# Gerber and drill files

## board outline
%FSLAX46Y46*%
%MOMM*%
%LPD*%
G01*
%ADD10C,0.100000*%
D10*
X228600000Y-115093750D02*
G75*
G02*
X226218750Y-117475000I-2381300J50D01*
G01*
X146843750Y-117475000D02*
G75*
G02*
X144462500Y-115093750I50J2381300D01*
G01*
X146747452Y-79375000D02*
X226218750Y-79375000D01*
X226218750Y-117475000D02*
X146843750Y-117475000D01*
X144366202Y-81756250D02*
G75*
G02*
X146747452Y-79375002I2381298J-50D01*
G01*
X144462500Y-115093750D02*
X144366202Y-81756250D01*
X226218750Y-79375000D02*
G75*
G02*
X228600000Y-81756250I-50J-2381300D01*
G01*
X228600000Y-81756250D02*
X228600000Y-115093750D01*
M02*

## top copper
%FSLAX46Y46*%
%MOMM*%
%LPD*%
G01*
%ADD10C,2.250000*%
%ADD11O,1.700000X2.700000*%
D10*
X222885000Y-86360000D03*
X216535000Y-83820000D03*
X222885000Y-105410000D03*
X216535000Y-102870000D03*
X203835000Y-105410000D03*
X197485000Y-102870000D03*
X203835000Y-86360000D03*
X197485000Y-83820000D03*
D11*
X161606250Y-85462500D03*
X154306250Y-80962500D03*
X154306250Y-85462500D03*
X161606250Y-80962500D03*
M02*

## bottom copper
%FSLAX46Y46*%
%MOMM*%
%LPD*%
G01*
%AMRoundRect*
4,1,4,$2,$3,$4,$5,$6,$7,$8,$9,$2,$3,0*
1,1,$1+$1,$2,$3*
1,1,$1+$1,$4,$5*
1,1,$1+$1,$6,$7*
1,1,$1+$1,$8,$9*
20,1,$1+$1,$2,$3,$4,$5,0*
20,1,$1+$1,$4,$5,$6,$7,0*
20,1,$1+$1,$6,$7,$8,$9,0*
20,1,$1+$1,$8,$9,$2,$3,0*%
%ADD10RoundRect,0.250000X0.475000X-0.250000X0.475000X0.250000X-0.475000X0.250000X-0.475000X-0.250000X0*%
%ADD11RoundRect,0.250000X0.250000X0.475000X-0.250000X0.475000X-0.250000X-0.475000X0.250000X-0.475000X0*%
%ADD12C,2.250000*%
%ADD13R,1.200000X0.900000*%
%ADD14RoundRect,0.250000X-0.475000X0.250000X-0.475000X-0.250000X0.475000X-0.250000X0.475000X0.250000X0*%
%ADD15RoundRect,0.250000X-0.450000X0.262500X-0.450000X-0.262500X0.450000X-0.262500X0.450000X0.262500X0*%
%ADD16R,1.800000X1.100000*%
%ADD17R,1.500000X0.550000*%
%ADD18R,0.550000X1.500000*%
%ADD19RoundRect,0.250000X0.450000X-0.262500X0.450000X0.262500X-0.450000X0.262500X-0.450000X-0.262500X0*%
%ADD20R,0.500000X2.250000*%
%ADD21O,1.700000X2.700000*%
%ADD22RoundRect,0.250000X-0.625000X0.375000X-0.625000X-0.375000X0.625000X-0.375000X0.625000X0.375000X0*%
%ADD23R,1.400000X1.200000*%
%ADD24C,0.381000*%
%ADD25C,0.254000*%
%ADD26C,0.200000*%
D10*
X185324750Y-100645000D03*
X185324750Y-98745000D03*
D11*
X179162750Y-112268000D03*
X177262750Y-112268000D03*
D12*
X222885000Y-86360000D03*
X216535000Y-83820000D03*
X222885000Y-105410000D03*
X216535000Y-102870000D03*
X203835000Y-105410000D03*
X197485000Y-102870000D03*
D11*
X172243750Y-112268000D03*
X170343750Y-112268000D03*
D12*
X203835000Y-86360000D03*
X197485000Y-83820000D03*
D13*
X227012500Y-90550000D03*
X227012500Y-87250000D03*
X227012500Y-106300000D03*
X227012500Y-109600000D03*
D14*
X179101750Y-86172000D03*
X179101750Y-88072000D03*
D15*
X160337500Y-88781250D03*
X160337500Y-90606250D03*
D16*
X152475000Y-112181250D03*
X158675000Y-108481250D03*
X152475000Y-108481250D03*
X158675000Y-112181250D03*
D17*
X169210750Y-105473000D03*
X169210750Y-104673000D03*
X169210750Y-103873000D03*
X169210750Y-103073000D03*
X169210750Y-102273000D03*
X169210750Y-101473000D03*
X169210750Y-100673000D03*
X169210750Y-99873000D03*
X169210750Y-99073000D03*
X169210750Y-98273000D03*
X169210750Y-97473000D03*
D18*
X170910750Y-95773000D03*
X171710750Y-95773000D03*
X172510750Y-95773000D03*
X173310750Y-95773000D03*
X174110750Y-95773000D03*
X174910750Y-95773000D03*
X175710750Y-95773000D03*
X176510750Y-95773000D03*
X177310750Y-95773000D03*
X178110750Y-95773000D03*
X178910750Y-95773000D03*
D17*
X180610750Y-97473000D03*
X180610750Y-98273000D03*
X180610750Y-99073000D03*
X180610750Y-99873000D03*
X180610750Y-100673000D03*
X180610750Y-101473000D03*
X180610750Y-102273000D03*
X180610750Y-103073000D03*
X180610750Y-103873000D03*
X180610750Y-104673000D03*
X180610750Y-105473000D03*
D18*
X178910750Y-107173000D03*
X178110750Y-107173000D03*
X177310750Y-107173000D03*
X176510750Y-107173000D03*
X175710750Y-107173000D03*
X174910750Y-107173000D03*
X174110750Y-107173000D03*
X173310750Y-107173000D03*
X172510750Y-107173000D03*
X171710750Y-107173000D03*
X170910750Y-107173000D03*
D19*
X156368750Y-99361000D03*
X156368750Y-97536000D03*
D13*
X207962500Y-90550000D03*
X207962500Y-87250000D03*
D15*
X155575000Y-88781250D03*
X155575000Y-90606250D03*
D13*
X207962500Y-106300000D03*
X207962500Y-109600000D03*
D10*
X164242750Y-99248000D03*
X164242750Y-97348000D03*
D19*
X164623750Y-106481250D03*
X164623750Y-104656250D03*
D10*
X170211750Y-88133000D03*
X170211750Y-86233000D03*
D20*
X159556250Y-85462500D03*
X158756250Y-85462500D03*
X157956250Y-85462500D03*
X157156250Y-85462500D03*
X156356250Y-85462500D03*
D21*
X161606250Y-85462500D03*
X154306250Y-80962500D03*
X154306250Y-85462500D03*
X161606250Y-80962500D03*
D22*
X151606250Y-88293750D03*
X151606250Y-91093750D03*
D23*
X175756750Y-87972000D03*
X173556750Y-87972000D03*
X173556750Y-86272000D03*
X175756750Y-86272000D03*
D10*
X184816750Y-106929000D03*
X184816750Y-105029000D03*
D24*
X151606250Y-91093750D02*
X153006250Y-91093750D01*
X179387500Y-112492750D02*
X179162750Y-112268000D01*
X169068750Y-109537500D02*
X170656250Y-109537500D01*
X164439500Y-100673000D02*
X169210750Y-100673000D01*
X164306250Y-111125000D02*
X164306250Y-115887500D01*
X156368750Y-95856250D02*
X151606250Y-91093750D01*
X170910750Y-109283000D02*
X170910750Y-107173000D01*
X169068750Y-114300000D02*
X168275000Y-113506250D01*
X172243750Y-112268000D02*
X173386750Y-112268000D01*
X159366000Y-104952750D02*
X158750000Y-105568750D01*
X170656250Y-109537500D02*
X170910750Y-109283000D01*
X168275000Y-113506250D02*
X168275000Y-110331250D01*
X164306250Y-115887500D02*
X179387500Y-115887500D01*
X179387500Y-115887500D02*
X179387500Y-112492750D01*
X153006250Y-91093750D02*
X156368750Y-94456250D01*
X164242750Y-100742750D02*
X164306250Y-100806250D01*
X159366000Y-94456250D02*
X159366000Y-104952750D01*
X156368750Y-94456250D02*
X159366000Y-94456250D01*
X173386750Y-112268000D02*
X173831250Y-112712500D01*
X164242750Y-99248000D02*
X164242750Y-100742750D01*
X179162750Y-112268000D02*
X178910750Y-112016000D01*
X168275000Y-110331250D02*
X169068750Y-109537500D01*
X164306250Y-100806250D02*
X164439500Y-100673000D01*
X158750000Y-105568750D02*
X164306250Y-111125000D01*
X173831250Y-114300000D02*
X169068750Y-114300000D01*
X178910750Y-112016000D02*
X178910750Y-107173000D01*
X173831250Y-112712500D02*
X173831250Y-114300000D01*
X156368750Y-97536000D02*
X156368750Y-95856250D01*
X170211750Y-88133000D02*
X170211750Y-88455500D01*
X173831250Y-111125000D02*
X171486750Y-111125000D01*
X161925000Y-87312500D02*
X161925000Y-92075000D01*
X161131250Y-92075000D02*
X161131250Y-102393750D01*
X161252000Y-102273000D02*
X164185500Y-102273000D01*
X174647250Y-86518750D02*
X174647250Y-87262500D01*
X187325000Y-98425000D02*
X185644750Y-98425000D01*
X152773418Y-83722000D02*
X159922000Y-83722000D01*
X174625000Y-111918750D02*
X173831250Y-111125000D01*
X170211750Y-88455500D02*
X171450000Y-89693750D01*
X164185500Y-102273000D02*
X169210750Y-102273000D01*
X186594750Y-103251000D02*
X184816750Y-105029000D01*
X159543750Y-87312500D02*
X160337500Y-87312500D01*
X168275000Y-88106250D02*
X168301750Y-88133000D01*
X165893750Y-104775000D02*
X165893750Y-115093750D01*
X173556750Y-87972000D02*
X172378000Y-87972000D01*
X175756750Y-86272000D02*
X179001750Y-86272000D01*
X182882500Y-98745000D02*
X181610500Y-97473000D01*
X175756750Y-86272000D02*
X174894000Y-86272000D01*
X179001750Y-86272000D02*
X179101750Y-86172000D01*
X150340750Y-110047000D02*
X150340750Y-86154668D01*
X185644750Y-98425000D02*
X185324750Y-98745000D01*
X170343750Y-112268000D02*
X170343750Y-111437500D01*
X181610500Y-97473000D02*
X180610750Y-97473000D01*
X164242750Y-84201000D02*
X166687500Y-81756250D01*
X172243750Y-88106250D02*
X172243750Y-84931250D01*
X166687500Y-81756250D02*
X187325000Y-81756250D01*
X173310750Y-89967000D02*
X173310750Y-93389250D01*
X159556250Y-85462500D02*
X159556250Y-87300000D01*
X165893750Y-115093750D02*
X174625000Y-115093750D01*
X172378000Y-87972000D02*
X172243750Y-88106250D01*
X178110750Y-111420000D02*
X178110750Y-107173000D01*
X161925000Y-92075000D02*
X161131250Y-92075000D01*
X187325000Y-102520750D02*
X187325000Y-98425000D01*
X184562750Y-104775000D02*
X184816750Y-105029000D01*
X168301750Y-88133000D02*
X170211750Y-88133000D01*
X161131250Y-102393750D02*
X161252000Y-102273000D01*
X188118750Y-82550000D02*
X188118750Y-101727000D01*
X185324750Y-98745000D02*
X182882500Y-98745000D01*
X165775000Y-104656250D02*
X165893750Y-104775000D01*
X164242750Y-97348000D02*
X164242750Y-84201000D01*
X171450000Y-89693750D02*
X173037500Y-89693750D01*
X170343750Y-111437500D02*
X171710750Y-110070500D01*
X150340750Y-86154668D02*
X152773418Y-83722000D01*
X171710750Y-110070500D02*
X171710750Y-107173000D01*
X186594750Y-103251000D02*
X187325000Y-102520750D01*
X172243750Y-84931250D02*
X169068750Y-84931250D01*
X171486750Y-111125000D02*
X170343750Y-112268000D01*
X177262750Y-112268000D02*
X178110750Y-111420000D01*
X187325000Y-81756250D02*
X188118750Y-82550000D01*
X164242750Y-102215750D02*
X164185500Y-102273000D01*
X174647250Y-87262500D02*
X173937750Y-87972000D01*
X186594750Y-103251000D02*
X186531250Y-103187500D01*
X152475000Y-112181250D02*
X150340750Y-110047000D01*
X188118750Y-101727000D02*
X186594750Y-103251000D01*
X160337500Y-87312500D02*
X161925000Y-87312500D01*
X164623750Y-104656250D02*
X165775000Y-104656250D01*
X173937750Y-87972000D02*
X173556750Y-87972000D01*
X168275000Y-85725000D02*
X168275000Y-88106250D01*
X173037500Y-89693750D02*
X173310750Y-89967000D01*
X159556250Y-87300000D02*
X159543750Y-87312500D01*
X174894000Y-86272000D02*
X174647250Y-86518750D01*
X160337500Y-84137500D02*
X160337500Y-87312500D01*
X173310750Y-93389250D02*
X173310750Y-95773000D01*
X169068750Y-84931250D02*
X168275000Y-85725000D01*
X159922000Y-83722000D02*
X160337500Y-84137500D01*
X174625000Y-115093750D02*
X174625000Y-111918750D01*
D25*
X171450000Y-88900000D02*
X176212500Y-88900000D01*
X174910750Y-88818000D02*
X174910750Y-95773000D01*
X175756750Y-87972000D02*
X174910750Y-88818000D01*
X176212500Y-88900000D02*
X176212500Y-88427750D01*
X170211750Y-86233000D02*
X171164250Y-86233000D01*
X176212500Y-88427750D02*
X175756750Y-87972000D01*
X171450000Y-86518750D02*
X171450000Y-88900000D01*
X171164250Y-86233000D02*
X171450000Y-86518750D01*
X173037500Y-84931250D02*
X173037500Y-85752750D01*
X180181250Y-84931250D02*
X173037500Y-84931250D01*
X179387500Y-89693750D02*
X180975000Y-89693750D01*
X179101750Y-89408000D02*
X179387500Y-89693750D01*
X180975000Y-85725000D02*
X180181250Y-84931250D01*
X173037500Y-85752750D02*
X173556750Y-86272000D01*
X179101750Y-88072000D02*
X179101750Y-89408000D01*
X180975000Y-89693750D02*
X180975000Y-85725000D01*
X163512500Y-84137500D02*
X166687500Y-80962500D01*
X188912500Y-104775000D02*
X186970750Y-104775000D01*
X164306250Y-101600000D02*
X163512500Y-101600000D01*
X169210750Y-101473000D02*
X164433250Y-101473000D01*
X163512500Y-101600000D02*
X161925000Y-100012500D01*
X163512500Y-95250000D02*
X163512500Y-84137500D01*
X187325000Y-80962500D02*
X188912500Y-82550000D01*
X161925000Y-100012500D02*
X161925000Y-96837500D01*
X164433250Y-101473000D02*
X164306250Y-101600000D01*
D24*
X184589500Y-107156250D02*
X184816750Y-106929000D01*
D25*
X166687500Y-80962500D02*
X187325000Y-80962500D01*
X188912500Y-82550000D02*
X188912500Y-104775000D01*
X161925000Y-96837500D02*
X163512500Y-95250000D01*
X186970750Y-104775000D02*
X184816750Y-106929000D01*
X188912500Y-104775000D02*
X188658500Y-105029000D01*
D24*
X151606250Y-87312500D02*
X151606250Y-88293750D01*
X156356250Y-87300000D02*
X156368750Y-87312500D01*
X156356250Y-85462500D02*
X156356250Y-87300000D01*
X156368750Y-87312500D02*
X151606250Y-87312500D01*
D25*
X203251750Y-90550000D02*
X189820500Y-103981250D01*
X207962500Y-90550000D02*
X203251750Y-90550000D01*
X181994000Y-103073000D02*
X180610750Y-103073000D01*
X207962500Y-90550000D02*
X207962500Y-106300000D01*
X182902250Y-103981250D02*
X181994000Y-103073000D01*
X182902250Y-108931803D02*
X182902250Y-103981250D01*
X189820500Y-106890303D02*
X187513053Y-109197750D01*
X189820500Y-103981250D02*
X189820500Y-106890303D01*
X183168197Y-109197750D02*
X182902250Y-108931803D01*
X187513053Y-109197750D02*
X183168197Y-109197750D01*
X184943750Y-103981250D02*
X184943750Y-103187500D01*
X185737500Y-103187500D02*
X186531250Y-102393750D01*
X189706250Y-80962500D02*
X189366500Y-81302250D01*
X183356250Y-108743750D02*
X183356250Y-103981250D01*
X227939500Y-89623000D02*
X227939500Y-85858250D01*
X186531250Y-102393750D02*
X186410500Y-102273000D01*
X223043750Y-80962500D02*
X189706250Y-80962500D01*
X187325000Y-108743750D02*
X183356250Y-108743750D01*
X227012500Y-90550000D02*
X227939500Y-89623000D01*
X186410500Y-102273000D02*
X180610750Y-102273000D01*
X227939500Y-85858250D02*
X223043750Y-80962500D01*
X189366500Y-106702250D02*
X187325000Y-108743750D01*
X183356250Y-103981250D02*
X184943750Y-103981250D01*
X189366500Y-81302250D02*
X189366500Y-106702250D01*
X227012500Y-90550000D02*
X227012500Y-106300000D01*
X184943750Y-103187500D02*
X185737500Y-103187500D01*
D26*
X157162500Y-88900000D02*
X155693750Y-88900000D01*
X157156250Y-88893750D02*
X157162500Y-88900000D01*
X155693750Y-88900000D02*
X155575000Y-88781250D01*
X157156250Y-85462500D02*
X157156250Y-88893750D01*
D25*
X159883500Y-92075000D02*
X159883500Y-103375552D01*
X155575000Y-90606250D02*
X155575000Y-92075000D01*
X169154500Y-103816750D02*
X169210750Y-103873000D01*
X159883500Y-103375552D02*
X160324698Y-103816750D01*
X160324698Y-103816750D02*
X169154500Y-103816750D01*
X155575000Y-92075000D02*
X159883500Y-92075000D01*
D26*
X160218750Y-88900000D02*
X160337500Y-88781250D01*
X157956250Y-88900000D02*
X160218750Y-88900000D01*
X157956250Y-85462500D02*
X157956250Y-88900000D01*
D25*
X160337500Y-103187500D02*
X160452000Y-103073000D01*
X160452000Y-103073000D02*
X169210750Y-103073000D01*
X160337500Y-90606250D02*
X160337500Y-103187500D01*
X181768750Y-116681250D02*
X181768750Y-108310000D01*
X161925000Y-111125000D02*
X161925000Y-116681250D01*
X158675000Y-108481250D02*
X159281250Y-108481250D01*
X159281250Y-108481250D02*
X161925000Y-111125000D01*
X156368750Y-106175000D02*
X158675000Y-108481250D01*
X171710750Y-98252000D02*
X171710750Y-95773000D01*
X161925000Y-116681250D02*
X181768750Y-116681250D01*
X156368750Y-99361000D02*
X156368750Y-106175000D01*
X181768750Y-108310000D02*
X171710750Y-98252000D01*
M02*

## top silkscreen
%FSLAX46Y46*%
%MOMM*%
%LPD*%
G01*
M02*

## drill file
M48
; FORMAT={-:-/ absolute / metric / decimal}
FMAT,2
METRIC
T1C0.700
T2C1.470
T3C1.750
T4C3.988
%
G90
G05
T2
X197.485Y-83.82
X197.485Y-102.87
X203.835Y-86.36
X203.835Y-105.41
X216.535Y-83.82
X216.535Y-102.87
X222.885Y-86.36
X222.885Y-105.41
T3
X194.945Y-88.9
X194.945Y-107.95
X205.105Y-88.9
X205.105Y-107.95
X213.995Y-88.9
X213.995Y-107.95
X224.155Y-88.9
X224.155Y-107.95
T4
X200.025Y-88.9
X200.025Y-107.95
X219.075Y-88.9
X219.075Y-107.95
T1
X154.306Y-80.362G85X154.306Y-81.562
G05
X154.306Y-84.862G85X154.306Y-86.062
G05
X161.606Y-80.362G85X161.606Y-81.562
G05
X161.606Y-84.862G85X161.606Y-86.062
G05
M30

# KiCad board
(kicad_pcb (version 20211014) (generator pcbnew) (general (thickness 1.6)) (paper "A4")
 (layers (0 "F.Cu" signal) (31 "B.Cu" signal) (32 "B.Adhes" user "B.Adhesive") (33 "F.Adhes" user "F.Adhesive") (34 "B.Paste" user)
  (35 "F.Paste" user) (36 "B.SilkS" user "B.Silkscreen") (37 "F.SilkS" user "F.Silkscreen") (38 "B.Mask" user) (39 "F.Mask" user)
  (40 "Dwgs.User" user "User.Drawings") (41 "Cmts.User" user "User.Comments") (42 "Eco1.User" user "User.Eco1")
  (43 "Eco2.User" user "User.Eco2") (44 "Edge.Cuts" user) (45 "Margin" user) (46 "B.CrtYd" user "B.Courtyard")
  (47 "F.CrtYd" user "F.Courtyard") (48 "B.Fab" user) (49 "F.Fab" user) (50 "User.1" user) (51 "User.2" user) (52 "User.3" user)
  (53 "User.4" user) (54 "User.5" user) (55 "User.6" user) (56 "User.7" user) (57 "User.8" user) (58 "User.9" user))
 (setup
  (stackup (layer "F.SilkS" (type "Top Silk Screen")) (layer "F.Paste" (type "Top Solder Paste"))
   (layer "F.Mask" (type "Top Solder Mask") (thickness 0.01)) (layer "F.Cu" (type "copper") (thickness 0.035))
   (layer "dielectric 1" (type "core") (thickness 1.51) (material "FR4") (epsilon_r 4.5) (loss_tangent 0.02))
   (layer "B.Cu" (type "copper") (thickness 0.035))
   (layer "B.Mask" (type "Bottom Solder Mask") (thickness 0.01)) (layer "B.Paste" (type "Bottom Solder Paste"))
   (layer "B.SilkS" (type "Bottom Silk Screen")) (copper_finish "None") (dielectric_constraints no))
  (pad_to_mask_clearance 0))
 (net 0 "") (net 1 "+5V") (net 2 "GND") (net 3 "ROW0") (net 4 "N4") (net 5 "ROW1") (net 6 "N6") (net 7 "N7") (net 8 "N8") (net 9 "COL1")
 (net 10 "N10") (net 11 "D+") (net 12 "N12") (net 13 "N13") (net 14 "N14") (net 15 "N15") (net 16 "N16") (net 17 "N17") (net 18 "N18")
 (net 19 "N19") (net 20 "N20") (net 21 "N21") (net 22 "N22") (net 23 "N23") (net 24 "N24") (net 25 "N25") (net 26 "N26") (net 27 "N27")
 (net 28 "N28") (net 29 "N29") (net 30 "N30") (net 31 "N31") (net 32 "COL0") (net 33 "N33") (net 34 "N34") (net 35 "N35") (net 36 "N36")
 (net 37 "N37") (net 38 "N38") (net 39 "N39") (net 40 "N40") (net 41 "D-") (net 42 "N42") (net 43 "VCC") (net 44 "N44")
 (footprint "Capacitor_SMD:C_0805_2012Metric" (layer "B.Cu") (at 185.32475 99.695 90)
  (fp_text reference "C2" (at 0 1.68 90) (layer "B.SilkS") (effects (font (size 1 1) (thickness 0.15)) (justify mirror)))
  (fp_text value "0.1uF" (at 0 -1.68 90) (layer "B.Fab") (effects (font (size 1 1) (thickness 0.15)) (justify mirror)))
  (pad "1" smd roundrect (at -0.95 0 90) (size 1 1.45) (layers "B.Cu" "B.Paste" "B.Mask") (roundrect_rratio 0.25) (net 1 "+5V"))
  (pad "2" smd roundrect (at 0.95 0 90) (size 1 1.45) (layers "B.Cu" "B.Paste" "B.Mask") (roundrect_rratio 0.25) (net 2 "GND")))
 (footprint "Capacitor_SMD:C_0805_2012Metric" (layer "B.Cu") (at 178.21275 112.268 180)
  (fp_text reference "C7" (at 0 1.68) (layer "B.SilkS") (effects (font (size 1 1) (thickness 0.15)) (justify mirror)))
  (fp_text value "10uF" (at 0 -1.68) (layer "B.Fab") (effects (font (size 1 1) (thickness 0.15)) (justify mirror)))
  (pad "1" smd roundrect (at -0.95 0 180) (size 1 1.45) (layers "B.Cu" "B.Paste" "B.Mask") (roundrect_rratio 0.25) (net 1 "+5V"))
  (pad "2" smd roundrect (at 0.95 0 180) (size 1 1.45) (layers "B.Cu" "B.Paste" "B.Mask") (roundrect_rratio 0.25) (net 2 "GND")))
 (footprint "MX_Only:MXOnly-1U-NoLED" (layer "B.Cu") (at 219.075 88.9 180)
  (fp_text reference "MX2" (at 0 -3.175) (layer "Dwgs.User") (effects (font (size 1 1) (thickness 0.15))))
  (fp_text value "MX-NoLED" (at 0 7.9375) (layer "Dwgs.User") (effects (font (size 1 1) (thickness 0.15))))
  (pad "" np_thru_hole circle locked (at 0 0 180) (size 3.9878 3.9878) (drill 3.9878) (layers *.Cu *.Mask))
  (pad "" np_thru_hole circle locked (at -5.08 0 131.9004) (size 1.75 1.75) (drill 1.75) (layers *.Cu *.Mask))
  (pad "" np_thru_hole circle locked (at 5.08 0 131.9004) (size 1.75 1.75) (drill 1.75) (layers *.Cu *.Mask))
  (pad "1" thru_hole circle locked (at -3.81 2.54 180) (size 2.25 2.25) (drill 1.47) (layers *.Cu "F.Mask") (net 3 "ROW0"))
  (pad "2" thru_hole circle locked (at 2.54 5.08 180) (size 2.25 2.25) (drill 1.47) (layers *.Cu "F.Mask") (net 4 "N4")))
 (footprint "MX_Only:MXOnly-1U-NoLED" (layer "B.Cu") (at 219.075 107.95 180)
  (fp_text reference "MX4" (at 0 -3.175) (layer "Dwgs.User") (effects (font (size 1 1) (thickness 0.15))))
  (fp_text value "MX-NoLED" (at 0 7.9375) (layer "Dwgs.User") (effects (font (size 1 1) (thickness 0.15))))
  (pad "" np_thru_hole circle locked (at -5.08 0 131.9004) (size 1.75 1.75) (drill 1.75) (layers *.Cu *.Mask))
  (pad "" np_thru_hole circle locked (at 0 0 180) (size 3.9878 3.9878) (drill 3.9878) (layers *.Cu *.Mask))
  (pad "" np_thru_hole circle locked (at 5.08 0 131.9004) (size 1.75 1.75) (drill 1.75) (layers *.Cu *.Mask))
  (pad "1" thru_hole circle locked (at -3.81 2.54 180) (size 2.25 2.25) (drill 1.47) (layers *.Cu "F.Mask") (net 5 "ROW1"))
  (pad "2" thru_hole circle locked (at 2.54 5.08 180) (size 2.25 2.25) (drill 1.47) (layers *.Cu "F.Mask") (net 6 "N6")))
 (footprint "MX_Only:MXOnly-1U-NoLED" (layer "B.Cu") (at 200.025 107.95 180)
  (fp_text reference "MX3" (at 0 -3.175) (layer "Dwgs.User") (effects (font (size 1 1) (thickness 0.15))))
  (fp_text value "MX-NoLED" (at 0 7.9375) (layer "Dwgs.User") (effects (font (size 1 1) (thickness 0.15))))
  (pad "" np_thru_hole circle locked (at 5.08 0 131.9004) (size 1.75 1.75) (drill 1.75) (layers *.Cu *.Mask))
  (pad "" np_thru_hole circle locked (at 0 0 180) (size 3.9878 3.9878) (drill 3.9878) (layers *.Cu *.Mask))
  (pad "" np_thru_hole circle locked (at -5.08 0 131.9004) (size 1.75 1.75) (drill 1.75) (layers *.Cu *.Mask))
  (pad "1" thru_hole circle locked (at -3.81 2.54 180) (size 2.25 2.25) (drill 1.47) (layers *.Cu "F.Mask") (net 5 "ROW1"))
  (pad "2" thru_hole circle locked (at 2.54 5.08 180) (size 2.25 2.25) (drill 1.47) (layers *.Cu "F.Mask") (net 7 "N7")))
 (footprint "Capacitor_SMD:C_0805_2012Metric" (layer "B.Cu") (at 171.29375 112.268 180)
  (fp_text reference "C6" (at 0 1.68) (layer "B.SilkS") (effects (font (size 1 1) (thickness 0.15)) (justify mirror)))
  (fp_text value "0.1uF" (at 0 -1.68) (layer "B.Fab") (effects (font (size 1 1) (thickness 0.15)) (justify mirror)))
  (pad "1" smd roundrect (at -0.95 0 180) (size 1 1.45) (layers "B.Cu" "B.Paste" "B.Mask") (roundrect_rratio 0.25) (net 1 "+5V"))
  (pad "2" smd roundrect (at 0.95 0 180) (size 1 1.45) (layers "B.Cu" "B.Paste" "B.Mask") (roundrect_rratio 0.25) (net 2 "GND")))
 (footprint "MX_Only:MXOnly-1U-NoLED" (layer "B.Cu") (at 200.025 88.9 180)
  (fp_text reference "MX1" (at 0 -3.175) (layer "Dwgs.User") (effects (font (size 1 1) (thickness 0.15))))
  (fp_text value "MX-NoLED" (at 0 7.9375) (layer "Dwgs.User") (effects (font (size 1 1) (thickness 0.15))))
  (pad "" np_thru_hole circle locked (at 5.08 0 131.9004) (size 1.75 1.75) (drill 1.75) (layers *.Cu *.Mask))
  (pad "" np_thru_hole circle locked (at -5.08 0 131.9004) (size 1.75 1.75) (drill 1.75) (layers *.Cu *.Mask))
  (pad "" np_thru_hole circle locked (at 0 0 180) (size 3.9878 3.9878) (drill 3.9878) (layers *.Cu *.Mask))
  (pad "1" thru_hole circle locked (at -3.81 2.54 180) (size 2.25 2.25) (drill 1.47) (layers *.Cu "F.Mask") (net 3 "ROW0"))
  (pad "2" thru_hole circle locked (at 2.54 5.08 180) (size 2.25 2.25) (drill 1.47) (layers *.Cu "F.Mask") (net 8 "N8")))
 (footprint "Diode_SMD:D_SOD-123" (layer "B.Cu") (at 227.0125 88.9 90)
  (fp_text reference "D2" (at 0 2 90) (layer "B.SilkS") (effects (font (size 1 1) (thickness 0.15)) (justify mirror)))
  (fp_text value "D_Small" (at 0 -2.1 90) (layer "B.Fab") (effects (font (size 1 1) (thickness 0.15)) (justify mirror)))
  (pad "1" smd rect (at -1.65 0 90) (size 0.9 1.2) (layers "B.Cu" "B.Paste" "B.Mask") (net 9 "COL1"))
  (pad "2" smd rect (at 1.65 0 90) (size 0.9 1.2) (layers "B.Cu" "B.Paste" "B.Mask") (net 4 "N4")))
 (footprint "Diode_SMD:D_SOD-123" (layer "B.Cu") (at 227.0125 107.95 -90)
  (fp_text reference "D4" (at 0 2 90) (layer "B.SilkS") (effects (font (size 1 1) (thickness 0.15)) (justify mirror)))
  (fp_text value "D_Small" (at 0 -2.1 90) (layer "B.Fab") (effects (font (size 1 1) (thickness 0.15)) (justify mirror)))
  (pad "1" smd rect (at -1.65 0 270) (size 0.9 1.2) (layers "B.Cu" "B.Paste" "B.Mask") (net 9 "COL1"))
  (pad "2" smd rect (at 1.65 0 270) (size 0.9 1.2) (layers "B.Cu" "B.Paste" "B.Mask") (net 6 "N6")))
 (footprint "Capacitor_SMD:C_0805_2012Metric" (layer "B.Cu") (at 179.10175 87.122 -90)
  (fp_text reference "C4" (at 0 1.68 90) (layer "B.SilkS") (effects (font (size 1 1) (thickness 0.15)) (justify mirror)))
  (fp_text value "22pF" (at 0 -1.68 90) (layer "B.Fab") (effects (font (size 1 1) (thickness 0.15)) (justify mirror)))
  (pad "1" smd roundrect (at -0.95 0 270) (size 1 1.45) (layers "B.Cu" "B.Paste" "B.Mask") (roundrect_rratio 0.25) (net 2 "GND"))
  (pad "2" smd roundrect (at 0.95 0 270) (size 1 1.45) (layers "B.Cu" "B.Paste" "B.Mask") (roundrect_rratio 0.25) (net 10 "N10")))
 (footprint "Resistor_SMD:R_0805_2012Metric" (layer "B.Cu") (at 160.3375 89.69375 -90)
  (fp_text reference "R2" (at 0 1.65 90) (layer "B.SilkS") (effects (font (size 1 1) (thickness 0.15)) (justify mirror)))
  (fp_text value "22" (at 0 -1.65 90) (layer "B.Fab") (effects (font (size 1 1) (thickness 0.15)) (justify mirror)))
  (pad "1" smd roundrect (at -0.9125 0 270) (size 1.025 1.4) (layers "B.Cu" "B.Paste" "B.Mask") (roundrect_rratio 0.243902) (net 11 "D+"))
  (pad "2" smd roundrect (at 0.9125 0 270) (size 1.025 1.4) (layers "B.Cu" "B.Paste" "B.Mask") (roundrect_rratio 0.243902) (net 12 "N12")))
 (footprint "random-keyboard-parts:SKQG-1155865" (layer "B.Cu") (at 155.575 110.33125 180)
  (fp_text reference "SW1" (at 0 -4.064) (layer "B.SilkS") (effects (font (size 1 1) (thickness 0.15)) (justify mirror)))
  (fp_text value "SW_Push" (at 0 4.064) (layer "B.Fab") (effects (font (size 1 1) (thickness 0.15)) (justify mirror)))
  (pad "1" smd rect locked (at 3.1 -1.85 180) (size 1.8 1.1) (layers "B.Cu" "B.Paste" "B.Mask") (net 2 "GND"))
  (pad "2" smd rect locked (at -3.1 1.85 180) (size 1.8 1.1) (layers "B.Cu" "B.Paste" "B.Mask") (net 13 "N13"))
  (pad "3" smd rect locked (at 3.1 1.85 180) (size 1.8 1.1) (layers "B.Cu" "B.Paste" "B.Mask"))
  (pad "4" smd rect locked (at -3.1 -1.85 180) (size 1.8 1.1) (layers "B.Cu" "B.Paste" "B.Mask")))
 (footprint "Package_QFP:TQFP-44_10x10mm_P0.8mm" (layer "B.Cu") (at 174.91075 101.473)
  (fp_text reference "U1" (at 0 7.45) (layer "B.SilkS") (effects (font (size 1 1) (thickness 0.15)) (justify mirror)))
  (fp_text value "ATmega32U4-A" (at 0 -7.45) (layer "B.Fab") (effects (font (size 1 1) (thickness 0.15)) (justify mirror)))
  (pad "1" smd rect (at -5.7 4) (size 1.5 0.55) (layers "B.Cu" "B.Paste" "B.Mask") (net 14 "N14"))
  (pad "2" smd rect (at -5.7 3.2) (size 1.5 0.55) (layers "B.Cu" "B.Paste" "B.Mask") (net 1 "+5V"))
  (pad "3" smd rect (at -5.7 2.4) (size 1.5 0.55) (layers "B.Cu" "B.Paste" "B.Mask") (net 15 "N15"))
  (pad "4" smd rect (at -5.7 1.6) (size 1.5 0.55) (layers "B.Cu" "B.Paste" "B.Mask") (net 12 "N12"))
  (pad "5" smd rect (at -5.7 0.8) (size 1.5 0.55) (layers "B.Cu" "B.Paste" "B.Mask") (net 2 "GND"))
  (pad "6" smd rect (at -5.7 0) (size 1.5 0.55) (layers "B.Cu" "B.Paste" "B.Mask") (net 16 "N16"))
  (pad "7" smd rect (at -5.7 -0.8) (size 1.5 0.55) (layers "B.Cu" "B.Paste" "B.Mask") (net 1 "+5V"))
  (pad "8" smd rect (at -5.7 -1.6) (size 1.5 0.55) (layers "B.Cu" "B.Paste" "B.Mask") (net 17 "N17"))
  (pad "9" smd rect (at -5.7 -2.4) (size 1.5 0.55) (layers "B.Cu" "B.Paste" "B.Mask") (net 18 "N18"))
  (pad "10" smd rect (at -5.7 -3.2) (size 1.5 0.55) (layers "B.Cu" "B.Paste" "B.Mask") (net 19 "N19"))
  (pad "11" smd rect (at -5.7 -4) (size 1.5 0.55) (layers "B.Cu" "B.Paste" "B.Mask") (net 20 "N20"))
  (pad "12" smd rect (at -4 -5.7 270) (size 1.5 0.55) (layers "B.Cu" "B.Paste" "B.Mask") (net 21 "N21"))
  (pad "13" smd rect (at -3.2 -5.7 270) (size 1.5 0.55) (layers "B.Cu" "B.Paste" "B.Mask") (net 13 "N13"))
  (pad "14" smd rect (at -2.4 -5.7 270) (size 1.5 0.55) (layers "B.Cu" "B.Paste" "B.Mask") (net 1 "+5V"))
  (pad "15" smd rect (at -1.6 -5.7 270) (size 1.5 0.55) (layers "B.Cu" "B.Paste" "B.Mask") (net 2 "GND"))
  (pad "16" smd rect (at -0.8 -5.7 270) (size 1.5 0.55) (layers "B.Cu" "B.Paste" "B.Mask") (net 10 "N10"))
  (pad "17" smd rect (at 0 -5.7 270) (size 1.5 0.55) (layers "B.Cu" "B.Paste" "B.Mask") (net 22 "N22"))
  (pad "18" smd rect (at 0.8 -5.7 270) (size 1.5 0.55) (layers "B.Cu" "B.Paste" "B.Mask") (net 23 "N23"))
  (pad "19" smd rect (at 1.6 -5.7 270) (size 1.5 0.55) (layers "B.Cu" "B.Paste" "B.Mask") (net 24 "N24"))
  (pad "20" smd rect (at 2.4 -5.7 270) (size 1.5 0.55) (layers "B.Cu" "B.Paste" "B.Mask") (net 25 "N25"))
  (pad "21" smd rect (at 3.2 -5.7 270) (size 1.5 0.55) (layers "B.Cu" "B.Paste" "B.Mask") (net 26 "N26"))
  (pad "22" smd rect (at 4 -5.7 270) (size 1.5 0.55) (layers "B.Cu" "B.Paste" "B.Mask") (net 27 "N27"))
  (pad "23" smd rect (at 5.7 -4) (size 1.5 0.55) (layers "B.Cu" "B.Paste" "B.Mask") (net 2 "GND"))
  (pad "24" smd rect (at 5.7 -3.2) (size 1.5 0.55) (layers "B.Cu" "B.Paste" "B.Mask") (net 1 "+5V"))
  (pad "25" smd rect (at 5.7 -2.4) (size 1.5 0.55) (layers "B.Cu" "B.Paste" "B.Mask") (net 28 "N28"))
  (pad "26" smd rect (at 5.7 -1.6) (size 1.5 0.55) (layers "B.Cu" "B.Paste" "B.Mask") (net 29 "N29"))
  (pad "27" smd rect (at 5.7 -0.8) (size 1.5 0.55) (layers "B.Cu" "B.Paste" "B.Mask") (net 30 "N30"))
  (pad "28" smd rect (at 5.7 0) (size 1.5 0.55) (layers "B.Cu" "B.Paste" "B.Mask") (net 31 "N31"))
  (pad "29" smd rect (at 5.7 0.8) (size 1.5 0.55) (layers "B.Cu" "B.Paste" "B.Mask") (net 9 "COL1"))
  (pad "30" smd rect (at 5.7 1.6) (size 1.5 0.55) (layers "B.Cu" "B.Paste" "B.Mask") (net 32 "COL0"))
  (pad "31" smd rect (at 5.7 2.4) (size 1.5 0.55) (layers "B.Cu" "B.Paste" "B.Mask") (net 5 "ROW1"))
  (pad "32" smd rect (at 5.7 3.2) (size 1.5 0.55) (layers "B.Cu" "B.Paste" "B.Mask") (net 3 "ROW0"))
  (pad "33" smd rect (at 5.7 4) (size 1.5 0.55) (layers "B.Cu" "B.Paste" "B.Mask") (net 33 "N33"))
  (pad "34" smd rect (at 4 5.7 270) (size 1.5 0.55) (layers "B.Cu" "B.Paste" "B.Mask") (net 1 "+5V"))
  (pad "35" smd rect (at 3.2 5.7 270) (size 1.5 0.55) (layers "B.Cu" "B.Paste" "B.Mask") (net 2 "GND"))
  (pad "36" smd rect (at 2.4 5.7 270) (size 1.5 0.55) (layers "B.Cu" "B.Paste" "B.Mask") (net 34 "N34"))
  (pad "37" smd rect (at 1.6 5.7 270) (size 1.5 0.55) (layers "B.Cu" "B.Paste" "B.Mask") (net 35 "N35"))
  (pad "38" smd rect (at 0.8 5.7 270) (size 1.5 0.55) (layers "B.Cu" "B.Paste" "B.Mask") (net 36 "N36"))
  (pad "39" smd rect (at 0 5.7 270) (size 1.5 0.55) (layers "B.Cu" "B.Paste" "B.Mask") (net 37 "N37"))
  (pad "40" smd rect (at -0.8 5.7 270) (size 1.5 0.55) (layers "B.Cu" "B.Paste" "B.Mask") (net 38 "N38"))
  (pad "41" smd rect (at -1.6 5.7 270) (size 1.5 0.55) (layers "B.Cu" "B.Paste" "B.Mask") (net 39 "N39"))
  (pad "42" smd rect (at -2.4 5.7 270) (size 1.5 0.55) (layers "B.Cu" "B.Paste" "B.Mask") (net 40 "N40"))
  (pad "43" smd rect (at -3.2 5.7 270) (size 1.5 0.55) (layers "B.Cu" "B.Paste" "B.Mask") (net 2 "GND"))
  (pad "44" smd rect (at -4 5.7 270) (size 1.5 0.55) (layers "B.Cu" "B.Paste" "B.Mask") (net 1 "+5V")))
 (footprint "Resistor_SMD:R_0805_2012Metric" (layer "B.Cu") (at 156.36875 98.4485 90)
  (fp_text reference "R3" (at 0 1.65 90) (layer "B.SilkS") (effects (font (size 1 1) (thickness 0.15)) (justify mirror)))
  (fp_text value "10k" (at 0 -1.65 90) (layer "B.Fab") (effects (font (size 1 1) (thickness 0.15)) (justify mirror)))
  (pad "1" smd roundrect (at -0.9125 0 90) (size 1.025 1.4) (layers "B.Cu" "B.Paste" "B.Mask") (roundrect_rratio 0.243902) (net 13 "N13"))
  (pad "2" smd roundrect (at 0.9125 0 90) (size 1.025 1.4) (layers "B.Cu" "B.Paste" "B.Mask") (roundrect_rratio 0.243902) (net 1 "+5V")))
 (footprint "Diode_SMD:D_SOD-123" (layer "B.Cu") (at 207.9625 88.9 90)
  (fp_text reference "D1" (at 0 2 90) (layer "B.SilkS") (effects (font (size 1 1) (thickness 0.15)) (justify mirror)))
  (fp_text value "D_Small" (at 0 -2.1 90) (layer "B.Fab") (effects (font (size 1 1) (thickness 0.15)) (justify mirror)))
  (pad "1" smd rect (at -1.65 0 90) (size 0.9 1.2) (layers "B.Cu" "B.Paste" "B.Mask") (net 32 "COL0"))
  (pad "2" smd rect (at 1.65 0 90) (size 0.9 1.2) (layers "B.Cu" "B.Paste" "B.Mask") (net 8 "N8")))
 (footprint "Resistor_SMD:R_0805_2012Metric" (layer "B.Cu") (at 155.575 89.69375 -90)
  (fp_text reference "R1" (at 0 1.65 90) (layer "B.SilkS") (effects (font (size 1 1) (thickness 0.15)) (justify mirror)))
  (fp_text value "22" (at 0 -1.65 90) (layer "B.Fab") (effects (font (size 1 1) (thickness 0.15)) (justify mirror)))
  (pad "1" smd roundrect (at -0.9125 0 270) (size 1.025 1.4) (layers "B.Cu" "B.Paste" "B.Mask") (roundrect_rratio 0.243902) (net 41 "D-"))
  (pad "2" smd roundrect (at 0.9125 0 270) (size 1.025 1.4) (layers "B.Cu" "B.Paste" "B.Mask") (roundrect_rratio 0.243902) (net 15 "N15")))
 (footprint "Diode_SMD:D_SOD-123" (layer "B.Cu") (at 207.9625 107.95 -90)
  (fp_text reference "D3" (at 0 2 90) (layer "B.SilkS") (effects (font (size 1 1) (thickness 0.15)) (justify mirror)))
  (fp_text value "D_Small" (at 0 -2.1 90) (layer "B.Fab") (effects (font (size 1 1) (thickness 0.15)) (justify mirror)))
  (pad "1" smd rect (at -1.65 0 270) (size 0.9 1.2) (layers "B.Cu" "B.Paste" "B.Mask") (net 32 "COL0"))
  (pad "2" smd rect (at 1.65 0 270) (size 0.9 1.2) (layers "B.Cu" "B.Paste" "B.Mask") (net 7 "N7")))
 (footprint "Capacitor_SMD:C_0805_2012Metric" (layer "B.Cu") (at 164.24275 98.298 90)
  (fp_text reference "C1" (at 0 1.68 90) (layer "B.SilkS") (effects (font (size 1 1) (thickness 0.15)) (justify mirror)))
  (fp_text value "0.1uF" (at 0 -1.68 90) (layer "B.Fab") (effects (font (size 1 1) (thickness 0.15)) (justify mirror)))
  (pad "1" smd roundrect (at -0.95 0 90) (size 1 1.45) (layers "B.Cu" "B.Paste" "B.Mask") (roundrect_rratio 0.25) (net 1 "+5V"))
  (pad "2" smd roundrect (at 0.95 0 90) (size 1 1.45) (layers "B.Cu" "B.Paste" "B.Mask") (roundrect_rratio 0.25) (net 2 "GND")))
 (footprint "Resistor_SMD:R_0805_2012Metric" (layer "B.Cu") (at 164.62375 105.56875 90)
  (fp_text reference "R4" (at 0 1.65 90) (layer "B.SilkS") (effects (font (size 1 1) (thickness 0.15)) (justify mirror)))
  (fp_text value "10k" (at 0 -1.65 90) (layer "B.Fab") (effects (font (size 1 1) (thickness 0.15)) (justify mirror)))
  (pad "1" smd roundrect (at -0.9125 0 90) (size 1.025 1.4) (layers "B.Cu" "B.Paste" "B.Mask") (roundrect_rratio 0.243902) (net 33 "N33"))
  (pad "2" smd roundrect (at 0.9125 0 90) (size 1.025 1.4) (layers "B.Cu" "B.Paste" "B.Mask") (roundrect_rratio 0.243902) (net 2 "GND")))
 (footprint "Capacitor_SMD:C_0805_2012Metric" (layer "B.Cu") (at 170.21175 87.183 90)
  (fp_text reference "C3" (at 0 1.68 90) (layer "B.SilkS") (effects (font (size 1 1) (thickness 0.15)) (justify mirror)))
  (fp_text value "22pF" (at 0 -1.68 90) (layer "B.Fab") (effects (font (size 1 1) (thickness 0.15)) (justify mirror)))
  (pad "1" smd roundrect (at -0.95 0 90) (size 1 1.45) (layers "B.Cu" "B.Paste" "B.Mask") (roundrect_rratio 0.25) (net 2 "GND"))
  (pad "2" smd roundrect (at 0.95 0 90) (size 1 1.45) (layers "B.Cu" "B.Paste" "B.Mask") (roundrect_rratio 0.25) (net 22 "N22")))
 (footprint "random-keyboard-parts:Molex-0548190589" (layer "B.Cu") (at 157.95625 80.9625 -90)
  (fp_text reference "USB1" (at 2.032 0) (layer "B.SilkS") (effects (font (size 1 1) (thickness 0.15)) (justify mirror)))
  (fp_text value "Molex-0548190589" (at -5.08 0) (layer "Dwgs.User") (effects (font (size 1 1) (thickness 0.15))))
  (pad "1" smd rect locked (at 4.5 -1.6 270) (size 2.25 0.5) (layers "B.Cu" "B.Paste" "B.Mask") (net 2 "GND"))
  (pad "2" smd rect locked (at 4.5 -0.8 270) (size 2.25 0.5) (layers "B.Cu" "B.Paste" "B.Mask") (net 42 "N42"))
  (pad "3" smd rect locked (at 4.5 0 270) (size 2.25 0.5) (layers "B.Cu" "B.Paste" "B.Mask") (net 11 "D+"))
  (pad "4" smd rect locked (at 4.5 0.8 270) (size 2.25 0.5) (layers "B.Cu" "B.Paste" "B.Mask") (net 41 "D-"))
  (pad "5" smd rect locked (at 4.5 1.6 270) (size 2.25 0.5) (layers "B.Cu" "B.Paste" "B.Mask") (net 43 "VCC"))
  (pad "6" thru_hole oval locked (at 4.5 -3.65 270) (size 2.7 1.7) (drill oval 1.9 0.7) (layers *.Cu *.Mask) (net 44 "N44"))
  (pad "6" thru_hole oval locked (at 0 3.65 270) (size 2.7 1.7) (drill oval 1.9 0.7) (layers *.Cu *.Mask) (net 44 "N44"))
  (pad "6" thru_hole oval locked (at 4.5 3.65 270) (size 2.7 1.7) (drill oval 1.9 0.7) (layers *.Cu *.Mask) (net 44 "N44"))
  (pad "6" thru_hole oval locked (at 0 -3.65 270) (size 2.7 1.7) (drill oval 1.9 0.7) (layers *.Cu *.Mask) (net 44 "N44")))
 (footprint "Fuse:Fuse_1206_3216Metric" (layer "B.Cu") (at 151.60625 89.69375 -90)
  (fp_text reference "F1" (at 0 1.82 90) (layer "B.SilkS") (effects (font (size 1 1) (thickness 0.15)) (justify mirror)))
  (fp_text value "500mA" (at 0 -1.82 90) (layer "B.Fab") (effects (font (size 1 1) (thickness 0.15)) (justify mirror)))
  (pad "1" smd roundrect (at -1.4 0 270) (size 1.25 1.75) (layers "B.Cu" "B.Paste" "B.Mask") (roundrect_rratio 0.2) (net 43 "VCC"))
  (pad "2" smd roundrect (at 1.4 0 270) (size 1.25 1.75) (layers "B.Cu" "B.Paste" "B.Mask") (roundrect_rratio 0.2) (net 1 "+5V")))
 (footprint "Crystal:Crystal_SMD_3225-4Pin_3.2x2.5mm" (layer "B.Cu") (at 174.65675 87.122 180)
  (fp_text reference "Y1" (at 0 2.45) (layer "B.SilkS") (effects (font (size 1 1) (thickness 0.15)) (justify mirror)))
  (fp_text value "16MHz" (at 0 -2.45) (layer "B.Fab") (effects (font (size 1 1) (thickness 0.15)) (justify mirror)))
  (pad "1" smd rect (at -1.1 -0.85 180) (size 1.4 1.2) (layers "B.Cu" "B.Paste" "B.Mask") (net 22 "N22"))
  (pad "2" smd rect (at 1.1 -0.85 180) (size 1.4 1.2) (layers "B.Cu" "B.Paste" "B.Mask") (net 2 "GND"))
  (pad "3" smd rect (at 1.1 0.85 180) (size 1.4 1.2) (layers "B.Cu" "B.Paste" "B.Mask") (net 10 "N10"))
  (pad "4" smd rect (at -1.1 0.85 180) (size 1.4 1.2) (layers "B.Cu" "B.Paste" "B.Mask") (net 2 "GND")))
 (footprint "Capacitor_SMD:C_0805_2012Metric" (layer "B.Cu") (at 184.81675 105.979 90)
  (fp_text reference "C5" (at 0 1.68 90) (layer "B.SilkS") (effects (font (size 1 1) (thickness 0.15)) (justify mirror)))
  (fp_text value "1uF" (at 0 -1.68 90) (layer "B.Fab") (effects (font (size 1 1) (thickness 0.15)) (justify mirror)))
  (pad "1" smd roundrect (at -0.95 0 90) (size 1 1.45) (layers "B.Cu" "B.Paste" "B.Mask") (roundrect_rratio 0.25) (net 16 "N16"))
  (pad "2" smd roundrect (at 0.95 0 90) (size 1 1.45) (layers "B.Cu" "B.Paste" "B.Mask") (roundrect_rratio 0.25) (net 2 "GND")))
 (gr_arc (start 228.6 115.09375) (mid 227.902548 116.777548) (end 226.21875 117.475) (layer "Edge.Cuts") (width 0.1))
 (gr_arc (start 146.84375 117.475) (mid 145.159952 116.777548) (end 144.4625 115.09375) (layer "Edge.Cuts") (width 0.1))
 (gr_line (start 146.747452 79.375) (end 226.21875 79.375) (layer "Edge.Cuts") (width 0.1))
 (gr_line (start 226.21875 117.475) (end 146.84375 117.475) (layer "Edge.Cuts") (width 0.1))
 (gr_arc (start 144.366202 81.75625) (mid 145.063654 80.072452) (end 146.747452 79.375) (layer "Edge.Cuts") (width 0.1))
 (gr_line (start 144.4625 115.09375) (end 144.366202 81.75625) (layer "Edge.Cuts") (width 0.1))
 (gr_arc (start 226.21875 79.375) (mid 227.902548 80.072452) (end 228.6 81.75625) (layer "Edge.Cuts") (width 0.1))
 (gr_line (start 228.6 81.75625) (end 228.6 115.09375) (layer "Edge.Cuts") (width 0.1))
 (segment (start 151.60625 91.09375) (end 153.00625 91.09375) (width 0.381) (layer "B.Cu") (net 1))
 (segment (start 179.3875 112.49275) (end 179.16275 112.268) (width 0.381) (layer "B.Cu") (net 1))
 (segment (start 169.06875 109.5375) (end 170.65625 109.5375) (width 0.381) (layer "B.Cu") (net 1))
 (segment (start 164.4395 100.673) (end 169.21075 100.673) (width 0.381) (layer "B.Cu") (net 1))
 (segment (start 164.30625 111.125) (end 164.30625 115.8875) (width 0.381) (layer "B.Cu") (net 1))
 (segment (start 156.36875 95.85625) (end 151.60625 91.09375) (width 0.381) (layer "B.Cu") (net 1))
 (segment (start 170.91075 109.283) (end 170.91075 107.173) (width 0.381) (layer "B.Cu") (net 1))
 (segment (start 169.06875 114.3) (end 168.275 113.50625) (width 0.381) (layer "B.Cu") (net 1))
 (segment (start 172.24375 112.268) (end 173.38675 112.268) (width 0.381) (layer "B.Cu") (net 1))
 (segment (start 159.366 104.95275) (end 158.75 105.56875) (width 0.381) (layer "B.Cu") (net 1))
 (segment (start 170.65625 109.5375) (end 170.91075 109.283) (width 0.381) (layer "B.Cu") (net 1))
 (segment (start 168.275 113.50625) (end 168.275 110.33125) (width 0.381) (layer "B.Cu") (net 1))
 (segment (start 164.30625 115.8875) (end 179.3875 115.8875) (width 0.381) (layer "B.Cu") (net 1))
 (segment (start 179.3875 115.8875) (end 179.3875 112.49275) (width 0.381) (layer "B.Cu") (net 1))
 (segment (start 153.00625 91.09375) (end 156.36875 94.45625) (width 0.381) (layer "B.Cu") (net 1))
 (segment (start 164.24275 100.74275) (end 164.30625 100.80625) (width 0.381) (layer "B.Cu") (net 1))
 (segment (start 159.366 94.45625) (end 159.366 104.95275) (width 0.381) (layer "B.Cu") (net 1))
 (segment (start 156.36875 94.45625) (end 159.366 94.45625) (width 0.381) (layer "B.Cu") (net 1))
 (segment (start 173.38675 112.268) (end 173.83125 112.7125) (width 0.381) (layer "B.Cu") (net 1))
 (segment (start 164.24275 99.248) (end 164.24275 100.74275) (width 0.381) (layer "B.Cu") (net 1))
 (segment (start 179.16275 112.268) (end 178.91075 112.016) (width 0.381) (layer "B.Cu") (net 1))
 (segment (start 168.275 110.33125) (end 169.06875 109.5375) (width 0.381) (layer "B.Cu") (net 1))
 (segment (start 164.30625 100.80625) (end 164.4395 100.673) (width 0.381) (layer "B.Cu") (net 1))
 (segment (start 158.75 105.56875) (end 164.30625 111.125) (width 0.381) (layer "B.Cu") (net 1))
 (segment (start 173.83125 114.3) (end 169.06875 114.3) (width 0.381) (layer "B.Cu") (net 1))
 (segment (start 178.91075 112.016) (end 178.91075 107.173) (width 0.381) (layer "B.Cu") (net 1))
 (segment (start 173.83125 112.7125) (end 173.83125 114.3) (width 0.381) (layer "B.Cu") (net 1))
 (segment (start 156.36875 97.536) (end 156.36875 95.85625) (width 0.381) (layer "B.Cu") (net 1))
 (segment (start 170.21175 88.133) (end 170.21175 88.4555) (width 0.381) (layer "B.Cu") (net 2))
 (segment (start 173.83125 111.125) (end 171.48675 111.125) (width 0.381) (layer "B.Cu") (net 2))
 (segment (start 161.925 87.3125) (end 161.925 92.075) (width 0.381) (layer "B.Cu") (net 2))
 (segment (start 161.13125 92.075) (end 161.13125 102.39375) (width 0.381) (layer "B.Cu") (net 2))
 (segment (start 161.252 102.273) (end 164.1855 102.273) (width 0.381) (layer "B.Cu") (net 2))
 (segment (start 174.64725 86.51875) (end 174.64725 87.2625) (width 0.381) (layer "B.Cu") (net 2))
 (segment (start 187.325 98.425) (end 185.64475 98.425) (width 0.381) (layer "B.Cu") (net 2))
 (segment (start 152.773418 83.722) (end 159.922 83.722) (width 0.381) (layer "B.Cu") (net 2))
 (segment (start 174.625 111.91875) (end 173.83125 111.125) (width 0.381) (layer "B.Cu") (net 2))
 (segment (start 170.21175 88.4555) (end 171.45 89.69375) (width 0.381) (layer "B.Cu") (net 2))
 (segment (start 164.1855 102.273) (end 169.21075 102.273) (width 0.381) (layer "B.Cu") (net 2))
 (segment (start 186.59475 103.251) (end 184.81675 105.029) (width 0.381) (layer "B.Cu") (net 2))
 (segment (start 159.54375 87.3125) (end 160.3375 87.3125) (width 0.381) (layer "B.Cu") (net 2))
 (segment (start 168.275 88.10625) (end 168.30175 88.133) (width 0.381) (layer "B.Cu") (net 2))
 (segment (start 165.89375 104.775) (end 165.89375 115.09375) (width 0.381) (layer "B.Cu") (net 2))
 (segment (start 173.55675 87.972) (end 172.378 87.972) (width 0.381) (layer "B.Cu") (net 2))
 (segment (start 175.75675 86.272) (end 179.00175 86.272) (width 0.381) (layer "B.Cu") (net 2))
 (segment (start 182.8825 98.745) (end 181.6105 97.473) (width 0.381) (layer "B.Cu") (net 2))
 (segment (start 175.75675 86.272) (end 174.894 86.272) (width 0.381) (layer "B.Cu") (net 2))
 (segment (start 179.00175 86.272) (end 179.10175 86.172) (width 0.381) (layer "B.Cu") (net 2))
 (segment (start 150.34075 110.047) (end 150.34075 86.154668) (width 0.381) (layer "B.Cu") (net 2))
 (segment (start 185.64475 98.425) (end 185.32475 98.745) (width 0.381) (layer "B.Cu") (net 2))
 (segment (start 170.34375 112.268) (end 170.34375 111.4375) (width 0.381) (layer "B.Cu") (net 2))
 (segment (start 181.6105 97.473) (end 180.61075 97.473) (width 0.381) (layer "B.Cu") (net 2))
 (segment (start 164.24275 84.201) (end 166.6875 81.75625) (width 0.381) (layer "B.Cu") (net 2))
 (segment (start 172.24375 88.10625) (end 172.24375 84.93125) (width 0.381) (layer "B.Cu") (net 2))
 (segment (start 166.6875 81.75625) (end 187.325 81.75625) (width 0.381) (layer "B.Cu") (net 2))
 (segment (start 173.31075 89.967) (end 173.31075 93.38925) (width 0.381) (layer "B.Cu") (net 2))
 (segment (start 159.55625 85.4625) (end 159.55625 87.3) (width 0.381) (layer "B.Cu") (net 2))
 (segment (start 165.89375 115.09375) (end 174.625 115.09375) (width 0.381) (layer "B.Cu") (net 2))
 (segment (start 172.378 87.972) (end 172.24375 88.10625) (width 0.381) (layer "B.Cu") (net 2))
 (segment (start 178.11075 111.42) (end 178.11075 107.173) (width 0.381) (layer "B.Cu") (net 2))
 (segment (start 161.925 92.075) (end 161.13125 92.075) (width 0.381) (layer "B.Cu") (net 2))
 (segment (start 187.325 102.52075) (end 187.325 98.425) (width 0.381) (layer "B.Cu") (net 2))
 (segment (start 184.56275 104.775) (end 184.81675 105.029) (width 0.381) (layer "B.Cu") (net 2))
 (segment (start 168.30175 88.133) (end 170.21175 88.133) (width 0.381) (layer "B.Cu") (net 2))
 (segment (start 161.13125 102.39375) (end 161.252 102.273) (width 0.381) (layer "B.Cu") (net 2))
 (segment (start 188.11875 82.55) (end 188.11875 101.727) (width 0.381) (layer "B.Cu") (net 2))
 (segment (start 185.32475 98.745) (end 182.8825 98.745) (width 0.381) (layer "B.Cu") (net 2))
 (segment (start 165.775 104.65625) (end 165.89375 104.775) (width 0.381) (layer "B.Cu") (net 2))
 (segment (start 164.24275 97.348) (end 164.24275 84.201) (width 0.381) (layer "B.Cu") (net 2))
 (segment (start 171.45 89.69375) (end 173.0375 89.69375) (width 0.381) (layer "B.Cu") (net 2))
 (segment (start 170.34375 111.4375) (end 171.71075 110.0705) (width 0.381) (layer "B.Cu") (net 2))
 (segment (start 150.34075 86.154668) (end 152.773418 83.722) (width 0.381) (layer "B.Cu") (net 2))
 (segment (start 171.71075 110.0705) (end 171.71075 107.173) (width 0.381) (layer "B.Cu") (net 2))
 (segment (start 186.59475 103.251) (end 187.325 102.52075) (width 0.381) (layer "B.Cu") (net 2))
 (segment (start 172.24375 84.93125) (end 169.06875 84.93125) (width 0.381) (layer "B.Cu") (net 2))
 (segment (start 171.48675 111.125) (end 170.34375 112.268) (width 0.381) (layer "B.Cu") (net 2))
 (segment (start 177.26275 112.268) (end 178.11075 111.42) (width 0.381) (layer "B.Cu") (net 2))
 (segment (start 187.325 81.75625) (end 188.11875 82.55) (width 0.381) (layer "B.Cu") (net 2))
 (segment (start 164.24275 102.21575) (end 164.1855 102.273) (width 0.381) (layer "B.Cu") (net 2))
 (segment (start 174.64725 87.2625) (end 173.93775 87.972) (width 0.381) (layer "B.Cu") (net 2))
 (segment (start 186.59475 103.251) (end 186.53125 103.1875) (width 0.381) (layer "B.Cu") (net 2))
 (segment (start 152.475 112.18125) (end 150.34075 110.047) (width 0.381) (layer "B.Cu") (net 2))
 (segment (start 188.11875 101.727) (end 186.59475 103.251) (width 0.381) (layer "B.Cu") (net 2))
 (segment (start 160.3375 87.3125) (end 161.925 87.3125) (width 0.381) (layer "B.Cu") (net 2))
 (segment (start 164.62375 104.65625) (end 165.775 104.65625) (width 0.381) (layer "B.Cu") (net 2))
 (segment (start 173.93775 87.972) (end 173.55675 87.972) (width 0.381) (layer "B.Cu") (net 2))
 (segment (start 168.275 85.725) (end 168.275 88.10625) (width 0.381) (layer "B.Cu") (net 2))
 (segment (start 173.0375 89.69375) (end 173.31075 89.967) (width 0.381) (layer "B.Cu") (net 2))
 (segment (start 159.55625 87.3) (end 159.54375 87.3125) (width 0.381) (layer "B.Cu") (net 2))
 (segment (start 174.894 86.272) (end 174.64725 86.51875) (width 0.381) (layer "B.Cu") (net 2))
 (segment (start 160.3375 84.1375) (end 160.3375 87.3125) (width 0.381) (layer "B.Cu") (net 2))
 (segment (start 173.31075 93.38925) (end 173.31075 95.773) (width 0.381) (layer "B.Cu") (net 2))
 (segment (start 169.06875 84.93125) (end 168.275 85.725) (width 0.381) (layer "B.Cu") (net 2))
 (segment (start 159.922 83.722) (end 160.3375 84.1375) (width 0.381) (layer "B.Cu") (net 2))
 (segment (start 174.625 115.09375) (end 174.625 111.91875) (width 0.381) (layer "B.Cu") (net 2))
 (segment (start 171.45 88.9) (end 176.2125 88.9) (width 0.254) (layer "B.Cu") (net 22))
 (segment (start 174.91075 88.818) (end 174.91075 95.773) (width 0.254) (layer "B.Cu") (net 22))
 (segment (start 175.75675 87.972) (end 174.91075 88.818) (width 0.254) (layer "B.Cu") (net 22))
 (segment (start 176.2125 88.9) (end 176.2125 88.42775) (width 0.254) (layer "B.Cu") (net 22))
 (segment (start 170.21175 86.233) (end 171.16425 86.233) (width 0.254) (layer "B.Cu") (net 22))
 (segment (start 176.2125 88.42775) (end 175.75675 87.972) (width 0.254) (layer "B.Cu") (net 22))
 (segment (start 171.45 86.51875) (end 171.45 88.9) (width 0.254) (layer "B.Cu") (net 22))
 (segment (start 171.16425 86.233) (end 171.45 86.51875) (width 0.254) (layer "B.Cu") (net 22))
 (segment (start 173.0375 84.93125) (end 173.0375 85.75275) (width 0.254) (layer "B.Cu") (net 10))
 (segment (start 180.18125 84.93125) (end 173.0375 84.93125) (width 0.254) (layer "B.Cu") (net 10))
 (segment (start 179.3875 89.69375) (end 180.975 89.69375) (width 0.254) (layer "B.Cu") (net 10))
 (segment (start 179.10175 89.408) (end 179.3875 89.69375) (width 0.254) (layer "B.Cu") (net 10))
 (segment (start 180.975 85.725) (end 180.18125 84.93125) (width 0.254) (layer "B.Cu") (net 10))
 (segment (start 173.0375 85.75275) (end 173.55675 86.272) (width 0.254) (layer "B.Cu") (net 10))
 (segment (start 179.10175 88.072) (end 179.10175 89.408) (width 0.254) (layer "B.Cu") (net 10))
 (segment (start 180.975 89.69375) (end 180.975 85.725) (width 0.254) (layer "B.Cu") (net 10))
 (segment (start 163.5125 84.1375) (end 166.6875 80.9625) (width 0.254) (layer "B.Cu") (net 16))
 (segment (start 188.9125 104.775) (end 186.97075 104.775) (width 0.254) (layer "B.Cu") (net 16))
 (segment (start 164.30625 101.6) (end 163.5125 101.6) (width 0.254) (layer "B.Cu") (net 16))
 (segment (start 169.21075 101.473) (end 164.43325 101.473) (width 0.254) (layer "B.Cu") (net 16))
 (segment (start 163.5125 101.6) (end 161.925 100.0125) (width 0.254) (layer "B.Cu") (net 16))
 (segment (start 163.5125 95.25) (end 163.5125 84.1375) (width 0.254) (layer "B.Cu") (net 16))
 (segment (start 187.325 80.9625) (end 188.9125 82.55) (width 0.254) (layer "B.Cu") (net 16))
 (segment (start 161.925 100.0125) (end 161.925 96.8375) (width 0.254) (layer "B.Cu") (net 16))
 (segment (start 164.43325 101.473) (end 164.30625 101.6) (width 0.254) (layer "B.Cu") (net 16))
 (segment (start 184.5895 107.15625) (end 184.81675 106.929) (width 0.381) (layer "B.Cu") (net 16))
 (segment (start 166.6875 80.9625) (end 187.325 80.9625) (width 0.254) (layer "B.Cu") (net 16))
 (segment (start 188.9125 82.55) (end 188.9125 104.775) (width 0.254) (layer "B.Cu") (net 16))
 (segment (start 161.925 96.8375) (end 163.5125 95.25) (width 0.254) (layer "B.Cu") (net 16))
 (segment (start 186.97075 104.775) (end 184.81675 106.929) (width 0.254) (layer "B.Cu") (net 16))
 (segment (start 188.9125 104.775) (end 188.6585 105.029) (width 0.254) (layer "B.Cu") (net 16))
 (segment (start 151.60625 87.3125) (end 151.60625 88.29375) (width 0.381) (layer "B.Cu") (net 43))
 (segment (start 156.35625 87.3) (end 156.36875 87.3125) (width 0.381) (layer "B.Cu") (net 43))
 (segment (start 156.35625 85.4625) (end 156.35625 87.3) (width 0.381) (layer "B.Cu") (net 43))
 (segment (start 156.36875 87.3125) (end 151.60625 87.3125) (width 0.381) (layer "B.Cu") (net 43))
 (segment (start 203.25175 90.55) (end 189.8205 103.98125) (width 0.254) (layer "B.Cu") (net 32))
 (segment (start 207.9625 90.55) (end 203.25175 90.55) (width 0.254) (layer "B.Cu") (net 32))
 (segment (start 181.994 103.073) (end 180.61075 103.073) (width 0.254) (layer "B.Cu") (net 32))
 (segment (start 207.9625 90.55) (end 207.9625 106.3) (width 0.254) (layer "B.Cu") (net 32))
 (segment (start 182.90225 103.98125) (end 181.994 103.073) (width 0.254) (layer "B.Cu") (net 32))
 (segment (start 182.90225 108.931803) (end 182.90225 103.98125) (width 0.254) (layer "B.Cu") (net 32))
 (segment (start 189.8205 106.890303) (end 187.513053 109.19775) (width 0.254) (layer "B.Cu") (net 32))
 (segment (start 189.8205 103.98125) (end 189.8205 106.890303) (width 0.254) (layer "B.Cu") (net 32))
 (segment (start 183.168197 109.19775) (end 182.90225 108.931803) (width 0.254) (layer "B.Cu") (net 32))
 (segment (start 187.513053 109.19775) (end 183.168197 109.19775) (width 0.254) (layer "B.Cu") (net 32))
 (segment (start 184.94375 103.98125) (end 184.94375 103.1875) (width 0.254) (layer "B.Cu") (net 9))
 (segment (start 185.7375 103.1875) (end 186.53125 102.39375) (width 0.254) (layer "B.Cu") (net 9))
 (segment (start 189.70625 80.9625) (end 189.3665 81.30225) (width 0.254) (layer "B.Cu") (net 9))
 (segment (start 183.35625 108.74375) (end 183.35625 103.98125) (width 0.254) (layer "B.Cu") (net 9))
 (segment (start 227.9395 89.623) (end 227.9395 85.85825) (width 0.254) (layer "B.Cu") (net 9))
 (segment (start 186.53125 102.39375) (end 186.4105 102.273) (width 0.254) (layer "B.Cu") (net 9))
 (segment (start 223.04375 80.9625) (end 189.70625 80.9625) (width 0.254) (layer "B.Cu") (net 9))
 (segment (start 187.325 108.74375) (end 183.35625 108.74375) (width 0.254) (layer "B.Cu") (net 9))
 (segment (start 227.0125 90.55) (end 227.9395 89.623) (width 0.254) (layer "B.Cu") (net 9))
 (segment (start 186.4105 102.273) (end 180.61075 102.273) (width 0.254) (layer "B.Cu") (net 9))
 (segment (start 227.9395 85.85825) (end 223.04375 80.9625) (width 0.254) (layer "B.Cu") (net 9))
 (segment (start 189.3665 106.70225) (end 187.325 108.74375) (width 0.254) (layer "B.Cu") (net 9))
 (segment (start 183.35625 103.98125) (end 184.94375 103.98125) (width 0.254) (layer "B.Cu") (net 9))
 (segment (start 189.3665 81.30225) (end 189.3665 106.70225) (width 0.254) (layer "B.Cu") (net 9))
 (segment (start 227.0125 90.55) (end 227.0125 106.3) (width 0.254) (layer "B.Cu") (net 9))
 (segment (start 184.94375 103.1875) (end 185.7375 103.1875) (width 0.254) (layer "B.Cu") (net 9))
 (segment (start 157.1625 88.9) (end 155.69375 88.9) (width 0.2) (layer "B.Cu") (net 41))
 (segment (start 157.15625 88.89375) (end 157.1625 88.9) (width 0.2) (layer "B.Cu") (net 41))
 (segment (start 155.69375 88.9) (end 155.575 88.78125) (width 0.2) (layer "B.Cu") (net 41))
 (segment (start 157.15625 85.4625) (end 157.15625 88.89375) (width 0.2) (layer "B.Cu") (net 41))
 (segment (start 159.8835 92.075) (end 159.8835 103.375552) (width 0.254) (layer "B.Cu") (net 15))
 (segment (start 155.575 90.60625) (end 155.575 92.075) (width 0.254) (layer "B.Cu") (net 15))
 (segment (start 169.1545 103.81675) (end 169.21075 103.873) (width 0.254) (layer "B.Cu") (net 15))
 (segment (start 159.8835 103.375552) (end 160.324698 103.81675) (width 0.254) (layer "B.Cu") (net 15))
 (segment (start 160.324698 103.81675) (end 169.1545 103.81675) (width 0.254) (layer "B.Cu") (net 15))
 (segment (start 155.575 92.075) (end 159.8835 92.075) (width 0.254) (layer "B.Cu") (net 15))
 (segment (start 160.21875 88.9) (end 160.3375 88.78125) (width 0.2) (layer "B.Cu") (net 11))
 (segment (start 157.95625 88.9) (end 160.21875 88.9) (width 0.2) (layer "B.Cu") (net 11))
 (segment (start 157.95625 85.4625) (end 157.95625 88.9) (width 0.2) (layer "B.Cu") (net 11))
 (segment (start 160.3375 103.1875) (end 160.452 103.073) (width 0.254) (layer "B.Cu") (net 12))
 (segment (start 160.452 103.073) (end 169.21075 103.073) (width 0.254) (layer "B.Cu") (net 12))
 (segment (start 160.3375 90.60625) (end 160.3375 103.1875) (width 0.254) (layer "B.Cu") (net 12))
 (segment (start 181.76875 116.68125) (end 181.76875 108.31) (width 0.254) (layer "B.Cu") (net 13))
 (segment (start 161.925 111.125) (end 161.925 116.68125) (width 0.254) (layer "B.Cu") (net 13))
 (segment (start 158.675 108.48125) (end 159.28125 108.48125) (width 0.254) (layer "B.Cu") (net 13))
 (segment (start 159.28125 108.48125) (end 161.925 111.125) (width 0.254) (layer "B.Cu") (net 13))
 (segment (start 156.36875 106.175) (end 158.675 108.48125) (width 0.254) (layer "B.Cu") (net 13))
 (segment (start 171.71075 98.252) (end 171.71075 95.773) (width 0.254) (layer "B.Cu") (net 13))
 (segment (start 161.925 116.68125) (end 181.76875 116.68125) (width 0.254) (layer "B.Cu") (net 13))
 (segment (start 156.36875 99.361) (end 156.36875 106.175) (width 0.254) (layer "B.Cu") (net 13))
 (segment (start 181.76875 108.31) (end 171.71075 98.252) (width 0.254) (layer "B.Cu") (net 13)))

